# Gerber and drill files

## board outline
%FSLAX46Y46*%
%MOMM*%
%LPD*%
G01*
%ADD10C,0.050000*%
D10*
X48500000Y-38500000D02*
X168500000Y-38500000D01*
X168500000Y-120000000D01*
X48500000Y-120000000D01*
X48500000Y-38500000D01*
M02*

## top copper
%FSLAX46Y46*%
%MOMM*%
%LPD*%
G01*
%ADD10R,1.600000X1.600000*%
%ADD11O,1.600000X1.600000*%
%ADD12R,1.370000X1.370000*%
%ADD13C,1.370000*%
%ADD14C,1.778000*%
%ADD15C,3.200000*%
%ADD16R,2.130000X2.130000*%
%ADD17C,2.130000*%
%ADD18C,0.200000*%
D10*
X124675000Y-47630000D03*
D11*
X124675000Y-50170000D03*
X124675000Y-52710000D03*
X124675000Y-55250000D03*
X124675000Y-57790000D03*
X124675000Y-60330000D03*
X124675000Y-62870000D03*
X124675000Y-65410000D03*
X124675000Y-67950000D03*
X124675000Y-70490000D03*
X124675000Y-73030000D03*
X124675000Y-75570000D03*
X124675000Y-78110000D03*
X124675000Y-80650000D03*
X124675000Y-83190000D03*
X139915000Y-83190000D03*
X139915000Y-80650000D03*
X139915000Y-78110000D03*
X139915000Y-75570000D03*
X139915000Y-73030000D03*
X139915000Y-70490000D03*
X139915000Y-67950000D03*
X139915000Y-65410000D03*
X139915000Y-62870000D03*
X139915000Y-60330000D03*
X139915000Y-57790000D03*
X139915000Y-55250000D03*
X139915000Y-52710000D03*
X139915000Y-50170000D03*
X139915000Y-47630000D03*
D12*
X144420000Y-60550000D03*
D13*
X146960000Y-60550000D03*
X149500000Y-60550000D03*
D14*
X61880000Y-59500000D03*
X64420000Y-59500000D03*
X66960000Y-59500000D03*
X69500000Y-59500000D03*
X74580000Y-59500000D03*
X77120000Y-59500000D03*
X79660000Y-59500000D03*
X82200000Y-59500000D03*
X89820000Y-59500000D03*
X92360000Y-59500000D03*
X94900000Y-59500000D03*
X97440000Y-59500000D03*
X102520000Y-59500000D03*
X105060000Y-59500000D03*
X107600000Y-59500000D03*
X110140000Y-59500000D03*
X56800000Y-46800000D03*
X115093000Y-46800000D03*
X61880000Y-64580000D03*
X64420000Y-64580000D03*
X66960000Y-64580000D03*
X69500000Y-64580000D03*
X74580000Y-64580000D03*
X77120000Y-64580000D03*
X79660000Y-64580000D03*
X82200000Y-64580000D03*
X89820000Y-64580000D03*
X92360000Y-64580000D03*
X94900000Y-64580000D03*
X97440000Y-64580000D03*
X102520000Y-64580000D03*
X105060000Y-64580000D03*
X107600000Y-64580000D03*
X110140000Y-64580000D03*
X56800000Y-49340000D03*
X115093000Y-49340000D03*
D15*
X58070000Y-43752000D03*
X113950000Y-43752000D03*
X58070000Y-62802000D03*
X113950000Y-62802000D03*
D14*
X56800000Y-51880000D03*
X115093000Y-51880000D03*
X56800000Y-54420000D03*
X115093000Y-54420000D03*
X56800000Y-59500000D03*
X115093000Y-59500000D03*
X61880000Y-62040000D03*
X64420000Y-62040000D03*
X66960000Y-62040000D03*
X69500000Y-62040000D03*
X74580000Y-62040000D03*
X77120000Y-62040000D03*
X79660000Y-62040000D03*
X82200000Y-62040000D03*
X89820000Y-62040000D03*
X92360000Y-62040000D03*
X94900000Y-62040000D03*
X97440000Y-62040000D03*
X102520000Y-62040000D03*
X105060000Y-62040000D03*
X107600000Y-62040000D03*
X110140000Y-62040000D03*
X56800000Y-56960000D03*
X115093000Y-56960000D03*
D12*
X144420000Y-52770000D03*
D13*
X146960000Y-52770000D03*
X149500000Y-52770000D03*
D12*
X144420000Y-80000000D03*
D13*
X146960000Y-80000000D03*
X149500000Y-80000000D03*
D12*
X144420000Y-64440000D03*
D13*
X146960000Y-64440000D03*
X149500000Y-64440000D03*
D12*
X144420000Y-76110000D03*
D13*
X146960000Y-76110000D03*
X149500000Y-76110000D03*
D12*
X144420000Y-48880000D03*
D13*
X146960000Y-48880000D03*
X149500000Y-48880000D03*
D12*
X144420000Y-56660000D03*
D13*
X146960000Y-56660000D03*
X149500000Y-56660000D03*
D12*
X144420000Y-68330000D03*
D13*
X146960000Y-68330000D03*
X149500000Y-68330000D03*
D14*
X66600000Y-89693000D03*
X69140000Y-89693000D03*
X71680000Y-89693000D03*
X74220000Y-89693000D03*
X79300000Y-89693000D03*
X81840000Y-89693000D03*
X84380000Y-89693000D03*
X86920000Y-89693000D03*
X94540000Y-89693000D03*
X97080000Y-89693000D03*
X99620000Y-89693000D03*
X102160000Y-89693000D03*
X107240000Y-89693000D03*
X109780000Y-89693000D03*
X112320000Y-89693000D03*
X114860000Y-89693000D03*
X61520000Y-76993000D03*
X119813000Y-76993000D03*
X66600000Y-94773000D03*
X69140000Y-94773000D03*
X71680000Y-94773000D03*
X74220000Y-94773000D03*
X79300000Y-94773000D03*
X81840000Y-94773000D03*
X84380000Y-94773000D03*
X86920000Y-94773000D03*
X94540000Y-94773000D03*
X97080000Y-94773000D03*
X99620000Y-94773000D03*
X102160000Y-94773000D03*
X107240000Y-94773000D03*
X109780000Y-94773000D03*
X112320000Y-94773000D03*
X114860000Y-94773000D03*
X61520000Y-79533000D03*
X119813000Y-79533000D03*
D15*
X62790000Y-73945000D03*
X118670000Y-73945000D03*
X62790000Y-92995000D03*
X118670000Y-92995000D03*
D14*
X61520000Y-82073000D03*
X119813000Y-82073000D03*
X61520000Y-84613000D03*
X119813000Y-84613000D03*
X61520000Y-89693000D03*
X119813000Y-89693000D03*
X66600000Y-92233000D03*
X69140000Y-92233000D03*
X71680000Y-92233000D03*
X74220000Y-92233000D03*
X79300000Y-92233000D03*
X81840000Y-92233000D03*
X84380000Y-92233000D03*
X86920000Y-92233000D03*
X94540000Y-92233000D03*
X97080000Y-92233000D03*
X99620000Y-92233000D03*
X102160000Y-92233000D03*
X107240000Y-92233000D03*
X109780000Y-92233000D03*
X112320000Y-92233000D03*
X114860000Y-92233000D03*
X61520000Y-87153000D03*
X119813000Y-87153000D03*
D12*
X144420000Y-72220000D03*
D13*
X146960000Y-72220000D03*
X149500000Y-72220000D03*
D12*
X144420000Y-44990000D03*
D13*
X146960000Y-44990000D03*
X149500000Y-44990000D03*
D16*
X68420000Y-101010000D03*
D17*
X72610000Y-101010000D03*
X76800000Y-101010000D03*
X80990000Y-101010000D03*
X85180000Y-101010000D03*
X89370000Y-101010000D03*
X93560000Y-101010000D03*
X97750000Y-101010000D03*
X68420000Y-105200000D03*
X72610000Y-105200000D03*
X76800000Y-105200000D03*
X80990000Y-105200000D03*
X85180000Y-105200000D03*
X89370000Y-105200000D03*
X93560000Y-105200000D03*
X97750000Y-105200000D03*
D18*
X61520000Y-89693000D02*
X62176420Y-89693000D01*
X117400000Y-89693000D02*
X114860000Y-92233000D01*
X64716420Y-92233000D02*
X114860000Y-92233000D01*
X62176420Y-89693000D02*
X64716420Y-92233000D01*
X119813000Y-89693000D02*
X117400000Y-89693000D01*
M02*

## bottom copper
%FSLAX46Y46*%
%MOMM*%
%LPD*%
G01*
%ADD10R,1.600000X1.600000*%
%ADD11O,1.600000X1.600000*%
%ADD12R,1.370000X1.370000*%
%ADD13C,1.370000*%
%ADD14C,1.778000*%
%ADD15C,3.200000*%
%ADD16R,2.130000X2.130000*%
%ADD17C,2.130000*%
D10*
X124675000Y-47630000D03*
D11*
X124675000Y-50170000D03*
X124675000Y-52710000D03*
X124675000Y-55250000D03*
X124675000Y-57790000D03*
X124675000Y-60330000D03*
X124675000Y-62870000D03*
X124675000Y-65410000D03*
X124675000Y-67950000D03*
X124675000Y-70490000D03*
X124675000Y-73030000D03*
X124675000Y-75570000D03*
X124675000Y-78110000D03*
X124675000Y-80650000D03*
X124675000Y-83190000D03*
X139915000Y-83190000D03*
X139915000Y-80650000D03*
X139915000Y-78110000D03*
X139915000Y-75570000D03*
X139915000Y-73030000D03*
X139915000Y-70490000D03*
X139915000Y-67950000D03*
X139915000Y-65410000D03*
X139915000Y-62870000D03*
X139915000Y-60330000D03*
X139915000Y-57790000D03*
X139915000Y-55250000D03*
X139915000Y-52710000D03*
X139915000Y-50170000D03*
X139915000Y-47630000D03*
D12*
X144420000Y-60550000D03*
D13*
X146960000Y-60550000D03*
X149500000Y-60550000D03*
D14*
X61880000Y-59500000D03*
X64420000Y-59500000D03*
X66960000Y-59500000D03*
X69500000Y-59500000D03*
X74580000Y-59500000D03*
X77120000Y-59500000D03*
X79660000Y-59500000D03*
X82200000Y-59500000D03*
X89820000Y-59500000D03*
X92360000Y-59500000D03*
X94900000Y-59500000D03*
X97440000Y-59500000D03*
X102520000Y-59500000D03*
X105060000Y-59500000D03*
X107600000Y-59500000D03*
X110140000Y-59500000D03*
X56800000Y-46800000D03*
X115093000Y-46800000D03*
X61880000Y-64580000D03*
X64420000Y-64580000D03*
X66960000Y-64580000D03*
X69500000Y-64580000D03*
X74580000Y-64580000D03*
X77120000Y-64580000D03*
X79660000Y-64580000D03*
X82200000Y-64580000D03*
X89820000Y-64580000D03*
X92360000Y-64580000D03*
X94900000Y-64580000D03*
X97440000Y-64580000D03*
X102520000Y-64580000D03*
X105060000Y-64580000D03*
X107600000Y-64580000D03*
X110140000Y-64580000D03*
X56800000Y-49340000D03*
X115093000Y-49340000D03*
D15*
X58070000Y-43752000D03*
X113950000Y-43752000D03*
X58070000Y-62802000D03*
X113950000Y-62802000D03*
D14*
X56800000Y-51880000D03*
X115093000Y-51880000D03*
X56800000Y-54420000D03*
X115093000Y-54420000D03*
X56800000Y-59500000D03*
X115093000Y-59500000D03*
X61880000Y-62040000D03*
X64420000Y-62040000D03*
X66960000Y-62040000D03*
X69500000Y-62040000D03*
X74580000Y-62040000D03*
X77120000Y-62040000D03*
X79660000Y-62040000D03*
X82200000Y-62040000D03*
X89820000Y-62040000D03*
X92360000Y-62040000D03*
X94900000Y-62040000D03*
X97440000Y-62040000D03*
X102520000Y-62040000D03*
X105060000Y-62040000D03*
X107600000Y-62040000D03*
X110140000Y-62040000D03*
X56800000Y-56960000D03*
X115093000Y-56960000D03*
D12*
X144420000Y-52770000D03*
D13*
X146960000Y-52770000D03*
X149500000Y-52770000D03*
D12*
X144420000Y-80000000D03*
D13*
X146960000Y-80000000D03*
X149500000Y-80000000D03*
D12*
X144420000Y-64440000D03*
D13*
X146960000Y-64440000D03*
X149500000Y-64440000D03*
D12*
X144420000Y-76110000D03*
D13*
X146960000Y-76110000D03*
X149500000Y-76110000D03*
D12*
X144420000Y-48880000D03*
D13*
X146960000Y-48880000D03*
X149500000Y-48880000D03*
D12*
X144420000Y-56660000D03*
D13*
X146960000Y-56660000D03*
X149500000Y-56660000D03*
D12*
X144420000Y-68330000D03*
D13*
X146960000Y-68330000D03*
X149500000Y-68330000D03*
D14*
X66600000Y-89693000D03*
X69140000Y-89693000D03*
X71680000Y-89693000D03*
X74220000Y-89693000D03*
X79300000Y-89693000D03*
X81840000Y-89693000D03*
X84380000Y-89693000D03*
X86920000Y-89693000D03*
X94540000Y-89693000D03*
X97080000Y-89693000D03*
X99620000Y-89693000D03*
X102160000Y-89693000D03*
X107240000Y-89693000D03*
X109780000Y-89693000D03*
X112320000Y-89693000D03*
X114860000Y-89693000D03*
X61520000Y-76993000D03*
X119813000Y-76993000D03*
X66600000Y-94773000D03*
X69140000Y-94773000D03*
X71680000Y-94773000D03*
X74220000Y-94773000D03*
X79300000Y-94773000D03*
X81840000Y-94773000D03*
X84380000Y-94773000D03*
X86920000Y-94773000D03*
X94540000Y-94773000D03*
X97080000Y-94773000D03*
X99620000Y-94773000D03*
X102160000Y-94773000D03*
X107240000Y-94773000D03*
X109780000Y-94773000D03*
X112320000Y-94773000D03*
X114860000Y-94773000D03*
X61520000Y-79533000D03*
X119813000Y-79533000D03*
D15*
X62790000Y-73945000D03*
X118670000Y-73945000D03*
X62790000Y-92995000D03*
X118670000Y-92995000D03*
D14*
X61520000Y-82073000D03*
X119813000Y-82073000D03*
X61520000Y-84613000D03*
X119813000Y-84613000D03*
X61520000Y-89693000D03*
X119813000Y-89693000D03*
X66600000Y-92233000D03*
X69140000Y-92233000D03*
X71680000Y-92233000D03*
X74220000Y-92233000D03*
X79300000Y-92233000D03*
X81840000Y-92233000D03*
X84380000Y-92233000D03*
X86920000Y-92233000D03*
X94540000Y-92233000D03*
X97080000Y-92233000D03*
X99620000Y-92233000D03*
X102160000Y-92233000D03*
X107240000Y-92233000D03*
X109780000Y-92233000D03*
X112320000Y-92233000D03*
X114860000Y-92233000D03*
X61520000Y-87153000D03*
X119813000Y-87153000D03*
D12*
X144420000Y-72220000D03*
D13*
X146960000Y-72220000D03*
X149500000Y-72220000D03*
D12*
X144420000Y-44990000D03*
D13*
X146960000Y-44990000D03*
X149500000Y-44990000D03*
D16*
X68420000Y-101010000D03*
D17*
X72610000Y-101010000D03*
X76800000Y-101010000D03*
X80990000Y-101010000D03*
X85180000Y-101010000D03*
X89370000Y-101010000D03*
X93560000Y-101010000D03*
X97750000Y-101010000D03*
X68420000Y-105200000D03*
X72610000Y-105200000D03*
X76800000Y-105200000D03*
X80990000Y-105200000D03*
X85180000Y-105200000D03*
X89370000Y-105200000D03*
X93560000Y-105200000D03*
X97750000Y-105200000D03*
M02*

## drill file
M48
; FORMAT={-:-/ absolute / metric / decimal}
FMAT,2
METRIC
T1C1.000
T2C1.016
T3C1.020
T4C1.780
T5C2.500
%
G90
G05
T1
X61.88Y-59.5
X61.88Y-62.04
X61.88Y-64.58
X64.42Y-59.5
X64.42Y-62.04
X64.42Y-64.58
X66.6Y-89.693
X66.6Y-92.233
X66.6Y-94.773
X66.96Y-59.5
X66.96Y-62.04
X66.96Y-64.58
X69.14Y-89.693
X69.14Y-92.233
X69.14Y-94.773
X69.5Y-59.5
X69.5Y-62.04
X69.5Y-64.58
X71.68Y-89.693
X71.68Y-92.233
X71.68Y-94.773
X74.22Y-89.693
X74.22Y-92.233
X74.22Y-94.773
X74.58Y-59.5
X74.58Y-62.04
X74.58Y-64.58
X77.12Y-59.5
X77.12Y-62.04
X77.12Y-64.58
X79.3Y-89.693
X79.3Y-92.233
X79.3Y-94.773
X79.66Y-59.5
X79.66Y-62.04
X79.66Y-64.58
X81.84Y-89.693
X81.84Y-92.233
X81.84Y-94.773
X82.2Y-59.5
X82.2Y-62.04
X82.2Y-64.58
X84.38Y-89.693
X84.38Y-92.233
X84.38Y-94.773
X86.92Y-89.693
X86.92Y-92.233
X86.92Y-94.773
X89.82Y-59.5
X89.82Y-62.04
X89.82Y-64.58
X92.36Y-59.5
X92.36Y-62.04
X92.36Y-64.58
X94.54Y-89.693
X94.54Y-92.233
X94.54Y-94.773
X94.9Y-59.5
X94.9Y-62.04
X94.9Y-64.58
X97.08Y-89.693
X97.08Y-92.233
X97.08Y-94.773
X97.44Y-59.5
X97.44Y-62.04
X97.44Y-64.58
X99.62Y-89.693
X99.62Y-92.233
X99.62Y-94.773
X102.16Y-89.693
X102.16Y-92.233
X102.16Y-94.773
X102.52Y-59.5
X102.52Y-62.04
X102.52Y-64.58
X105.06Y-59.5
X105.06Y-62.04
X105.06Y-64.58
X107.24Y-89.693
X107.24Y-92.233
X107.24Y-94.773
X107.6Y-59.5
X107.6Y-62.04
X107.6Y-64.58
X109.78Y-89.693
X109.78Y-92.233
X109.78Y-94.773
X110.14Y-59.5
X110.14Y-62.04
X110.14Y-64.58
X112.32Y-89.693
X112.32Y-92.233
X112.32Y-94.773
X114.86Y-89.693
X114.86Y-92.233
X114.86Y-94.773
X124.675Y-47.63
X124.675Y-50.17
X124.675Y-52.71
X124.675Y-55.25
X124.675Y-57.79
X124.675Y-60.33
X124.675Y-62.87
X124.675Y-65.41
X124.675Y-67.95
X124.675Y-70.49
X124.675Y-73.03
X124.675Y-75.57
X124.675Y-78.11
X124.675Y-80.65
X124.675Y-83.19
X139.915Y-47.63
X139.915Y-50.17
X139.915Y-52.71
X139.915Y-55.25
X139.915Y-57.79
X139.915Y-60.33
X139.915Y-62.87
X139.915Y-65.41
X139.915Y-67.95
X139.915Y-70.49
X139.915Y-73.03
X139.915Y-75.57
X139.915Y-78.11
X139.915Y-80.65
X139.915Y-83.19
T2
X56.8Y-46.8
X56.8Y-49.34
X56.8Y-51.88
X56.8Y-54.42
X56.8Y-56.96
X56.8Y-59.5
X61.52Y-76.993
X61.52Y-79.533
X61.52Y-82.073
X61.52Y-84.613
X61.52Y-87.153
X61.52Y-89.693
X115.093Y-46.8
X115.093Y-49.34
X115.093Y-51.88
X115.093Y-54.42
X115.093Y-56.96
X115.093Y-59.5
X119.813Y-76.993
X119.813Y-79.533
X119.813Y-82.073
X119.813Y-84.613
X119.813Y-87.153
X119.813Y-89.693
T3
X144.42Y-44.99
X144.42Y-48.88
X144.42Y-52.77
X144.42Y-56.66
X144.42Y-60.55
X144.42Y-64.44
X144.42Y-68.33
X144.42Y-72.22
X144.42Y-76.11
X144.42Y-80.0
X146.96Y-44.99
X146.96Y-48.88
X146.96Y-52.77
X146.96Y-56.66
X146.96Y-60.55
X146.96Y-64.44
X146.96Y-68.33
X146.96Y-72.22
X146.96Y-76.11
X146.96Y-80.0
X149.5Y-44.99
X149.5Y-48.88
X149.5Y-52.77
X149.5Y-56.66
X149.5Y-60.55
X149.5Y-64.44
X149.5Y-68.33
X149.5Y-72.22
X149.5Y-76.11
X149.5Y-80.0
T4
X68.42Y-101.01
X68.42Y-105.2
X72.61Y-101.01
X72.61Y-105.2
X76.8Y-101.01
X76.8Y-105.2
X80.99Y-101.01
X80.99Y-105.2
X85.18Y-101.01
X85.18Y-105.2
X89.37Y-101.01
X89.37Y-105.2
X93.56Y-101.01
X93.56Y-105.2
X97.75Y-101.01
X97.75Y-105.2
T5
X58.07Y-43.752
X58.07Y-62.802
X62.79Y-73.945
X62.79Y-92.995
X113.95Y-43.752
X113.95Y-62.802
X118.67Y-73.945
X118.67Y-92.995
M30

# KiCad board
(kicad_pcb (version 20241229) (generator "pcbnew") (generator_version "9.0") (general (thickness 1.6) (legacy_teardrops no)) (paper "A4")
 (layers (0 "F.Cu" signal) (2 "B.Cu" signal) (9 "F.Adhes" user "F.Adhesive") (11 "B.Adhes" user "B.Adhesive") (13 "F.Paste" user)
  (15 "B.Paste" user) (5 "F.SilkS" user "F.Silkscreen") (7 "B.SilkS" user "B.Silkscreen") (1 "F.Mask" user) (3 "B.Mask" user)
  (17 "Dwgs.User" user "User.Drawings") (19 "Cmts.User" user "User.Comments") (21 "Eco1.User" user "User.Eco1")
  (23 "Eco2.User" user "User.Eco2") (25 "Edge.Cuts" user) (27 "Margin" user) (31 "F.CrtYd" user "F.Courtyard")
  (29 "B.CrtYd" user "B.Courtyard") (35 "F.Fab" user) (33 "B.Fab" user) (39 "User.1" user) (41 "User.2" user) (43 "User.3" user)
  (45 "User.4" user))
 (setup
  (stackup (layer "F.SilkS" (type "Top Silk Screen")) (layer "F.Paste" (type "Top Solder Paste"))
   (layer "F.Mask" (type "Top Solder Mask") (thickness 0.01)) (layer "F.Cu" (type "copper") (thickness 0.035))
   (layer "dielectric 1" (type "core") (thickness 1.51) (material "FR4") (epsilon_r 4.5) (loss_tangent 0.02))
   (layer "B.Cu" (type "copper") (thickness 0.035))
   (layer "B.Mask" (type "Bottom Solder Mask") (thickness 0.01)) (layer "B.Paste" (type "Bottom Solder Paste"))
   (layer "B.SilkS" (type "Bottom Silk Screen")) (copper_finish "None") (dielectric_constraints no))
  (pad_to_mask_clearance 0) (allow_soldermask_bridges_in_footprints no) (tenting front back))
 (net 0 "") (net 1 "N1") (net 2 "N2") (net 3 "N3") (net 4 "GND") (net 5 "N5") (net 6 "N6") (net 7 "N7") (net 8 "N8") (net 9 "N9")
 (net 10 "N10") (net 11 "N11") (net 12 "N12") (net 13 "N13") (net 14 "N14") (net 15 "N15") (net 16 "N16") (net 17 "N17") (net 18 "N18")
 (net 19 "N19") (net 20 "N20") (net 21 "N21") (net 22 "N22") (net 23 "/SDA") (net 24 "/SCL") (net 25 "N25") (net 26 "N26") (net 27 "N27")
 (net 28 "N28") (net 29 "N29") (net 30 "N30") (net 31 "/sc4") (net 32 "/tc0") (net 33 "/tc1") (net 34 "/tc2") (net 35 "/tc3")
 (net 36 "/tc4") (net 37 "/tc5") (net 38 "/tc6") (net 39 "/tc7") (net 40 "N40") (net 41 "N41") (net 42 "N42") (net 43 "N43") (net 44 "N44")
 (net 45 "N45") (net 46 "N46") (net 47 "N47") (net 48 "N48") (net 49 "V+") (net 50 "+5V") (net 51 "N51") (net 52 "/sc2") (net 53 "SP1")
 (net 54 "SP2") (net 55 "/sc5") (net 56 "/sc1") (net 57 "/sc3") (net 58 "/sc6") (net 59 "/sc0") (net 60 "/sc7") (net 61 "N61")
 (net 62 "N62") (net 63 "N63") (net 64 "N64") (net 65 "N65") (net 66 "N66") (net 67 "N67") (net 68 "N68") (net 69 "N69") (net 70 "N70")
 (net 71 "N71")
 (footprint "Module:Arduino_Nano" (layer "F.Cu") (at 124.675 47.63)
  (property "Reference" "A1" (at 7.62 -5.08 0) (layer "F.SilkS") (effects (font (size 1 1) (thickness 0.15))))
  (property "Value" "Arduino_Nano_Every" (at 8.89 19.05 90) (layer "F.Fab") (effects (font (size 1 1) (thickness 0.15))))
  (pad "1" thru_hole rect (at 0 0) (size 1.6 1.6) (drill 1) (layers "*.Cu" "*.Mask") (remove_unused_layers no) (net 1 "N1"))
  (pad "2" thru_hole oval (at 0 2.54) (size 1.6 1.6) (drill 1) (layers "*.Cu" "*.Mask") (remove_unused_layers no) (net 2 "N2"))
  (pad "3" thru_hole oval (at 0 5.08) (size 1.6 1.6) (drill 1) (layers "*.Cu" "*.Mask") (remove_unused_layers no) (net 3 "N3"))
  (pad "4" thru_hole oval (at 0 7.62) (size 1.6 1.6) (drill 1) (layers "*.Cu" "*.Mask") (remove_unused_layers no) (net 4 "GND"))
  (pad "5" thru_hole oval (at 0 10.16) (size 1.6 1.6) (drill 1) (layers "*.Cu" "*.Mask") (remove_unused_layers no) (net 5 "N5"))
  (pad "6" thru_hole oval (at 0 12.7) (size 1.6 1.6) (drill 1) (layers "*.Cu" "*.Mask") (remove_unused_layers no) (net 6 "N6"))
  (pad "7" thru_hole oval (at 0 15.24) (size 1.6 1.6) (drill 1) (layers "*.Cu" "*.Mask") (remove_unused_layers no) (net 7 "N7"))
  (pad "8" thru_hole oval (at 0 17.78) (size 1.6 1.6) (drill 1) (layers "*.Cu" "*.Mask") (remove_unused_layers no) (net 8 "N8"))
  (pad "9" thru_hole oval (at 0 20.32) (size 1.6 1.6) (drill 1) (layers "*.Cu" "*.Mask") (remove_unused_layers no) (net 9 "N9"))
  (pad "10" thru_hole oval (at 0 22.86) (size 1.6 1.6) (drill 1) (layers "*.Cu" "*.Mask") (remove_unused_layers no) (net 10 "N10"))
  (pad "11" thru_hole oval (at 0 25.4) (size 1.6 1.6) (drill 1) (layers "*.Cu" "*.Mask") (remove_unused_layers no) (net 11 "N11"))
  (pad "12" thru_hole oval (at 0 27.94) (size 1.6 1.6) (drill 1) (layers "*.Cu" "*.Mask") (remove_unused_layers no) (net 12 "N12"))
  (pad "13" thru_hole oval (at 0 30.48) (size 1.6 1.6) (drill 1) (layers "*.Cu" "*.Mask") (remove_unused_layers no) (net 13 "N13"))
  (pad "14" thru_hole oval (at 0 33.02) (size 1.6 1.6) (drill 1) (layers "*.Cu" "*.Mask") (remove_unused_layers no) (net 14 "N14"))
  (pad "15" thru_hole oval (at 0 35.56) (size 1.6 1.6) (drill 1) (layers "*.Cu" "*.Mask") (remove_unused_layers no) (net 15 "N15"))
  (pad "16" thru_hole oval (at 15.24 35.56) (size 1.6 1.6) (drill 1) (layers "*.Cu" "*.Mask") (remove_unused_layers no) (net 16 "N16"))
  (pad "17" thru_hole oval (at 15.24 33.02) (size 1.6 1.6) (drill 1) (layers "*.Cu" "*.Mask") (remove_unused_layers no) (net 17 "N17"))
  (pad "18" thru_hole oval (at 15.24 30.48) (size 1.6 1.6) (drill 1) (layers "*.Cu" "*.Mask") (remove_unused_layers no) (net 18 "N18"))
  (pad "19" thru_hole oval (at 15.24 27.94) (size 1.6 1.6) (drill 1) (layers "*.Cu" "*.Mask") (remove_unused_layers no) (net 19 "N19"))
  (pad "20" thru_hole oval (at 15.24 25.4) (size 1.6 1.6) (drill 1) (layers "*.Cu" "*.Mask") (remove_unused_layers no) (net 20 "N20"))
  (pad "21" thru_hole oval (at 15.24 22.86) (size 1.6 1.6) (drill 1) (layers "*.Cu" "*.Mask") (remove_unused_layers no) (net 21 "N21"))
  (pad "22" thru_hole oval (at 15.24 20.32) (size 1.6 1.6) (drill 1) (layers "*.Cu" "*.Mask") (remove_unused_layers no) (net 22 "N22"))
  (pad "23" thru_hole oval (at 15.24 17.78) (size 1.6 1.6) (drill 1) (layers "*.Cu" "*.Mask") (remove_unused_layers no) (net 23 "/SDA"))
  (pad "24" thru_hole oval (at 15.24 15.24) (size 1.6 1.6) (drill 1) (layers "*.Cu" "*.Mask") (remove_unused_layers no) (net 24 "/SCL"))
  (pad "25" thru_hole oval (at 15.24 12.7) (size 1.6 1.6) (drill 1) (layers "*.Cu" "*.Mask") (remove_unused_layers no) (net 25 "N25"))
  (pad "26" thru_hole oval (at 15.24 10.16) (size 1.6 1.6) (drill 1) (layers "*.Cu" "*.Mask") (remove_unused_layers no) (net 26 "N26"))
  (pad "27" thru_hole oval (at 15.24 7.62) (size 1.6 1.6) (drill 1) (layers "*.Cu" "*.Mask") (remove_unused_layers no) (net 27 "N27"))
  (pad "28" thru_hole oval (at 15.24 5.08) (size 1.6 1.6) (drill 1) (layers "*.Cu" "*.Mask") (remove_unused_layers no) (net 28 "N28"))
  (pad "29" thru_hole oval (at 15.24 2.54) (size 1.6 1.6) (drill 1) (layers "*.Cu" "*.Mask") (remove_unused_layers no) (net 4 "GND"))
  (pad "30" thru_hole oval (at 15.24 0) (size 1.6 1.6) (drill 1) (layers "*.Cu" "*.Mask") (remove_unused_layers no) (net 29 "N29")))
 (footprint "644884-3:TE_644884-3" (layer "F.Cu") (at 144.42 60.55)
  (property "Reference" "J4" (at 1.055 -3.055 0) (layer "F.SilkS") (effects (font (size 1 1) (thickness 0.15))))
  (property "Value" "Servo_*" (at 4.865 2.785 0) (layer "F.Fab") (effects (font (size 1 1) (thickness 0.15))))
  (pad "1" thru_hole rect (at 0 0) (size 1.37 1.37) (drill 1.02) (layers "*.Cu" "*.Mask") (remove_unused_layers no) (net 4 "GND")
   (solder_mask_margin 0.102))
  (pad "2" thru_hole circle (at 2.54 0) (size 1.37 1.37) (drill 1.02) (layers "*.Cu" "*.Mask") (remove_unused_layers no) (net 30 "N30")
   (solder_mask_margin 0.102))
  (pad "3" thru_hole circle (at 5.08 0) (size 1.37 1.37) (drill 1.02) (layers "*.Cu" "*.Mask") (remove_unused_layers no) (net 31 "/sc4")
   (solder_mask_margin 0.102)))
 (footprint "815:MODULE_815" (layer "F.Cu") (at 86.01 53.277)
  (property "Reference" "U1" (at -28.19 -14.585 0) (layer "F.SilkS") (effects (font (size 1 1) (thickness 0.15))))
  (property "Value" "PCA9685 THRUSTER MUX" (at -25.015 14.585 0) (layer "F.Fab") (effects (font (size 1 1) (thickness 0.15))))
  (pad "0" thru_hole circle (at -24.13 6.223) (size 1.778 1.778) (drill 1) (layers "*.Cu" "*.Mask") (remove_unused_layers no)
   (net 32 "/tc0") (solder_mask_margin 0.102))
  (pad "1" thru_hole circle (at -21.59 6.223) (size 1.778 1.778) (drill 1) (layers "*.Cu" "*.Mask") (remove_unused_layers no)
   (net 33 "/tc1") (solder_mask_margin 0.102))
  (pad "2" thru_hole circle (at -19.05 6.223) (size 1.778 1.778) (drill 1) (layers "*.Cu" "*.Mask") (remove_unused_layers no)
   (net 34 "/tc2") (solder_mask_margin 0.102))
  (pad "3" thru_hole circle (at -16.51 6.223) (size 1.778 1.778) (drill 1) (layers "*.Cu" "*.Mask") (remove_unused_layers no)
   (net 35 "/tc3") (solder_mask_margin 0.102))
  (pad "4" thru_hole circle (at -11.43 6.223) (size 1.778 1.778) (drill 1) (layers "*.Cu" "*.Mask") (remove_unused_layers no)
   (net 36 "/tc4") (solder_mask_margin 0.102))
  (pad "5" thru_hole circle (at -8.89 6.223) (size 1.778 1.778) (drill 1) (layers "*.Cu" "*.Mask") (remove_unused_layers no) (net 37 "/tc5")
   (solder_mask_margin 0.102))
  (pad "6" thru_hole circle (at -6.35 6.223) (size 1.778 1.778) (drill 1) (layers "*.Cu" "*.Mask") (remove_unused_layers no) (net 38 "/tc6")
   (solder_mask_margin 0.102))
  (pad "7" thru_hole circle (at -3.81 6.223) (size 1.778 1.778) (drill 1) (layers "*.Cu" "*.Mask") (remove_unused_layers no) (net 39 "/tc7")
   (solder_mask_margin 0.102))
  (pad "8" thru_hole circle (at 3.81 6.223) (size 1.778 1.778) (drill 1) (layers "*.Cu" "*.Mask") (remove_unused_layers no) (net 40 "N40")
   (solder_mask_margin 0.102))
  (pad "9" thru_hole circle (at 6.35 6.223) (size 1.778 1.778) (drill 1) (layers "*.Cu" "*.Mask") (remove_unused_layers no) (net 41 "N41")
   (solder_mask_margin 0.102))
  (pad "10" thru_hole circle (at 8.89 6.223) (size 1.778 1.778) (drill 1) (layers "*.Cu" "*.Mask") (remove_unused_layers no) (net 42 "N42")
   (solder_mask_margin 0.102))
  (pad "11" thru_hole circle (at 11.43 6.223) (size 1.778 1.778) (drill 1) (layers "*.Cu" "*.Mask") (remove_unused_layers no) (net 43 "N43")
   (solder_mask_margin 0.102))
  (pad "12" thru_hole circle (at 16.51 6.223) (size 1.778 1.778) (drill 1) (layers "*.Cu" "*.Mask") (remove_unused_layers no) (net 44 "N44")
   (solder_mask_margin 0.102))
  (pad "13" thru_hole circle (at 19.05 6.223) (size 1.778 1.778) (drill 1) (layers "*.Cu" "*.Mask") (remove_unused_layers no) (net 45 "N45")
   (solder_mask_margin 0.102))
  (pad "14" thru_hole circle (at 21.59 6.223) (size 1.778 1.778) (drill 1) (layers "*.Cu" "*.Mask") (remove_unused_layers no) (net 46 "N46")
   (solder_mask_margin 0.102))
  (pad "15" thru_hole circle (at 24.13 6.223) (size 1.778 1.778) (drill 1) (layers "*.Cu" "*.Mask") (remove_unused_layers no) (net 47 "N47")
   (solder_mask_margin 0.102))
  (pad "GND_1" thru_hole circle (at -29.21 -6.477) (size 1.778 1.778) (drill 1.016) (layers "*.Cu" "*.Mask") (remove_unused_layers no)
   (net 4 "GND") (solder_mask_margin 0.102))
  (pad "GND_2" thru_hole circle (at 29.083 -6.477) (size 1.778 1.778) (drill 1.016) (layers "*.Cu" "*.Mask") (remove_unused_layers no)
   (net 4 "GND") (solder_mask_margin 0.102))
  (pad "GND_3" thru_hole circle (at -24.13 11.303) (size 1.778 1.778) (drill 1) (layers "*.Cu" "*.Mask") (remove_unused_layers no)
   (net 4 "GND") (solder_mask_margin 0.102))
  (pad "GND_4" thru_hole circle (at -21.59 11.303) (size 1.778 1.778) (drill 1) (layers "*.Cu" "*.Mask") (remove_unused_layers no)
   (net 4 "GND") (solder_mask_margin 0.102))
  (pad "GND_5" thru_hole circle (at -19.05 11.303) (size 1.778 1.778) (drill 1) (layers "*.Cu" "*.Mask") (remove_unused_layers no)
   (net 4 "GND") (solder_mask_margin 0.102))
  (pad "GND_6" thru_hole circle (at -16.51 11.303) (size 1.778 1.778) (drill 1) (layers "*.Cu" "*.Mask") (remove_unused_layers no)
   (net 4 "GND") (solder_mask_margin 0.102))
  (pad "GND_7" thru_hole circle (at -11.43 11.303) (size 1.778 1.778) (drill 1) (layers "*.Cu" "*.Mask") (remove_unused_layers no)
   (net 4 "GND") (solder_mask_margin 0.102))
  (pad "GND_8" thru_hole circle (at -8.89 11.303) (size 1.778 1.778) (drill 1) (layers "*.Cu" "*.Mask") (remove_unused_layers no)
   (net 4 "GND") (solder_mask_margin 0.102))
  (pad "GND_9" thru_hole circle (at -6.35 11.303) (size 1.778 1.778) (drill 1) (layers "*.Cu" "*.Mask") (remove_unused_layers no)
   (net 4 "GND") (solder_mask_margin 0.102))
  (pad "GND_10" thru_hole circle (at -3.81 11.303) (size 1.778 1.778) (drill 1) (layers "*.Cu" "*.Mask") (remove_unused_layers no)
   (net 4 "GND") (solder_mask_margin 0.102))
  (pad "GND_11" thru_hole circle (at 3.81 11.303) (size 1.778 1.778) (drill 1) (layers "*.Cu" "*.Mask") (remove_unused_layers no)
   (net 4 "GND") (solder_mask_margin 0.102))
  (pad "GND_12" thru_hole circle (at 6.35 11.303) (size 1.778 1.778) (drill 1) (layers "*.Cu" "*.Mask") (remove_unused_layers no)
   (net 4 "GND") (solder_mask_margin 0.102))
  (pad "GND_13" thru_hole circle (at 8.89 11.303) (size 1.778 1.778) (drill 1) (layers "*.Cu" "*.Mask") (remove_unused_layers no)
   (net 4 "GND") (solder_mask_margin 0.102))
  (pad "GND_14" thru_hole circle (at 11.43 11.303) (size 1.778 1.778) (drill 1) (layers "*.Cu" "*.Mask") (remove_unused_layers no)
   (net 4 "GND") (solder_mask_margin 0.102))
  (pad "GND_15" thru_hole circle (at 16.51 11.303) (size 1.778 1.778) (drill 1) (layers "*.Cu" "*.Mask") (remove_unused_layers no)
   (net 4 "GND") (solder_mask_margin 0.102))
  (pad "GND_16" thru_hole circle (at 19.05 11.303) (size 1.778 1.778) (drill 1) (layers "*.Cu" "*.Mask") (remove_unused_layers no)
   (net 4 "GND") (solder_mask_margin 0.102))
  (pad "GND_17" thru_hole circle (at 21.59 11.303) (size 1.778 1.778) (drill 1) (layers "*.Cu" "*.Mask") (remove_unused_layers no)
   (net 4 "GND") (solder_mask_margin 0.102))
  (pad "GND_18" thru_hole circle (at 24.13 11.303) (size 1.778 1.778) (drill 1) (layers "*.Cu" "*.Mask") (remove_unused_layers no)
   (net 4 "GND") (solder_mask_margin 0.102))
  (pad "OE_1" thru_hole circle (at -29.21 -3.937) (size 1.778 1.778) (drill 1.016) (layers "*.Cu" "*.Mask") (remove_unused_layers no)
   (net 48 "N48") (solder_mask_margin 0.102))
  (pad "OE_2" thru_hole circle (at 29.083 -3.937) (size 1.778 1.778) (drill 1.016) (layers "*.Cu" "*.Mask") (remove_unused_layers no)
   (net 48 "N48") (solder_mask_margin 0.102))
  (pad "S1" thru_hole circle (at -27.94 -9.525) (size 3.2 3.2) (drill 2.5) (layers "*.Cu" "*.Mask") (remove_unused_layers no)
   (solder_mask_margin 0.102))
  (pad "S2" thru_hole circle (at 27.94 -9.525) (size 3.2 3.2) (drill 2.5) (layers "*.Cu" "*.Mask") (remove_unused_layers no)
   (solder_mask_margin 0.102))
  (pad "S3" thru_hole circle (at -27.94 9.525) (size 3.2 3.2) (drill 2.5) (layers "*.Cu" "*.Mask") (remove_unused_layers no)
   (solder_mask_margin 0.102))
  (pad "S4" thru_hole circle (at 27.94 9.525) (size 3.2 3.2) (drill 2.5) (layers "*.Cu" "*.Mask") (remove_unused_layers no)
   (solder_mask_margin 0.102))
  (pad "SCL_1" thru_hole circle (at -29.21 -1.397) (size 1.778 1.778) (drill 1.016) (layers "*.Cu" "*.Mask") (remove_unused_layers no)
   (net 24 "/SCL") (solder_mask_margin 0.102))
  (pad "SCL_2" thru_hole circle (at 29.083 -1.397) (size 1.778 1.778) (drill 1.016) (layers "*.Cu" "*.Mask") (remove_unused_layers no)
   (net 24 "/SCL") (solder_mask_margin 0.102))
  (pad "SDA_1" thru_hole circle (at -29.21 1.143) (size 1.778 1.778) (drill 1.016) (layers "*.Cu" "*.Mask") (remove_unused_layers no)
   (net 23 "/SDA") (solder_mask_margin 0.102))
  (pad "SDA_2" thru_hole circle (at 29.083 1.143) (size 1.778 1.778) (drill 1.016) (layers "*.Cu" "*.Mask") (remove_unused_layers no)
   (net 23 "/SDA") (solder_mask_margin 0.102))
  (pad "V+_1" thru_hole circle (at -29.21 6.223) (size 1.778 1.778) (drill 1.016) (layers "*.Cu" "*.Mask") (remove_unused_layers no)
   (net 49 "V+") (solder_mask_margin 0.102))
  (pad "V+_2" thru_hole circle (at 29.083 6.223) (size 1.778 1.778) (drill 1.016) (layers "*.Cu" "*.Mask") (remove_unused_layers no)
   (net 49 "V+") (solder_mask_margin 0.102))
  (pad "V+_3" thru_hole circle (at -24.13 8.763) (size 1.778 1.778) (drill 1) (layers "*.Cu" "*.Mask") (remove_unused_layers no)
   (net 49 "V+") (solder_mask_margin 0.102))
  (pad "V+_4" thru_hole circle (at -21.59 8.763) (size 1.778 1.778) (drill 1) (layers "*.Cu" "*.Mask") (remove_unused_layers no)
   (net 49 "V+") (solder_mask_margin 0.102))
  (pad "V+_5" thru_hole circle (at -19.05 8.763) (size 1.778 1.778) (drill 1) (layers "*.Cu" "*.Mask") (remove_unused_layers no)
   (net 49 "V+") (solder_mask_margin 0.102))
  (pad "V+_6" thru_hole circle (at -16.51 8.763) (size 1.778 1.778) (drill 1) (layers "*.Cu" "*.Mask") (remove_unused_layers no)
   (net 49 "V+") (solder_mask_margin 0.102))
  (pad "V+_7" thru_hole circle (at -11.43 8.763) (size 1.778 1.778) (drill 1) (layers "*.Cu" "*.Mask") (remove_unused_layers no)
   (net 49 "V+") (solder_mask_margin 0.102))
  (pad "V+_8" thru_hole circle (at -8.89 8.763) (size 1.778 1.778) (drill 1) (layers "*.Cu" "*.Mask") (remove_unused_layers no)
   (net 49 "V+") (solder_mask_margin 0.102))
  (pad "V+_9" thru_hole circle (at -6.35 8.763) (size 1.778 1.778) (drill 1) (layers "*.Cu" "*.Mask") (remove_unused_layers no)
   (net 49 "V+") (solder_mask_margin 0.102))
  (pad "V+_10" thru_hole circle (at -3.81 8.763) (size 1.778 1.778) (drill 1) (layers "*.Cu" "*.Mask") (remove_unused_layers no)
   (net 49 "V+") (solder_mask_margin 0.102))
  (pad "V+_11" thru_hole circle (at 3.81 8.763) (size 1.778 1.778) (drill 1) (layers "*.Cu" "*.Mask") (remove_unused_layers no)
   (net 49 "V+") (solder_mask_margin 0.102))
  (pad "V+_12" thru_hole circle (at 6.35 8.763) (size 1.778 1.778) (drill 1) (layers "*.Cu" "*.Mask") (remove_unused_layers no)
   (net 49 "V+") (solder_mask_margin 0.102))
  (pad "V+_13" thru_hole circle (at 8.89 8.763) (size 1.778 1.778) (drill 1) (layers "*.Cu" "*.Mask") (remove_unused_layers no)
   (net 49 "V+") (solder_mask_margin 0.102))
  (pad "V+_14" thru_hole circle (at 11.43 8.763) (size 1.778 1.778) (drill 1) (layers "*.Cu" "*.Mask") (remove_unused_layers no)
   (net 49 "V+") (solder_mask_margin 0.102))
  (pad "V+_15" thru_hole circle (at 16.51 8.763) (size 1.778 1.778) (drill 1) (layers "*.Cu" "*.Mask") (remove_unused_layers no)
   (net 49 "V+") (solder_mask_margin 0.102))
  (pad "V+_16" thru_hole circle (at 19.05 8.763) (size 1.778 1.778) (drill 1) (layers "*.Cu" "*.Mask") (remove_unused_layers no)
   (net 49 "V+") (solder_mask_margin 0.102))
  (pad "V+_17" thru_hole circle (at 21.59 8.763) (size 1.778 1.778) (drill 1) (layers "*.Cu" "*.Mask") (remove_unused_layers no)
   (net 49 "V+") (solder_mask_margin 0.102))
  (pad "V+_18" thru_hole circle (at 24.13 8.763) (size 1.778 1.778) (drill 1) (layers "*.Cu" "*.Mask") (remove_unused_layers no)
   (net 49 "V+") (solder_mask_margin 0.102))
  (pad "VCC_1" thru_hole circle (at -29.21 3.683) (size 1.778 1.778) (drill 1.016) (layers "*.Cu" "*.Mask") (remove_unused_layers no)
   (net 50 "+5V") (solder_mask_margin 0.102))
  (pad "VCC_2" thru_hole circle (at 29.083 3.683) (size 1.778 1.778) (drill 1.016) (layers "*.Cu" "*.Mask") (remove_unused_layers no)
   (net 50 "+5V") (solder_mask_margin 0.102)))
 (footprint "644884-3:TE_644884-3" (layer "F.Cu") (at 144.42 52.77)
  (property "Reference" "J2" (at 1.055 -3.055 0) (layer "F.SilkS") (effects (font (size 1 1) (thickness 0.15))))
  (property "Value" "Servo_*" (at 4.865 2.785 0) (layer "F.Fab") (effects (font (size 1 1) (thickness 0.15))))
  (pad "1" thru_hole rect (at 0 0) (size 1.37 1.37) (drill 1.02) (layers "*.Cu" "*.Mask") (remove_unused_layers no) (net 4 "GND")
   (solder_mask_margin 0.102))
  (pad "2" thru_hole circle (at 2.54 0) (size 1.37 1.37) (drill 1.02) (layers "*.Cu" "*.Mask") (remove_unused_layers no) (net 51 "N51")
   (solder_mask_margin 0.102))
  (pad "3" thru_hole circle (at 5.08 0) (size 1.37 1.37) (drill 1.02) (layers "*.Cu" "*.Mask") (remove_unused_layers no) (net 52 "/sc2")
   (solder_mask_margin 0.102)))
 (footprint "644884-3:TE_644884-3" (layer "F.Cu") (at 144.42 80)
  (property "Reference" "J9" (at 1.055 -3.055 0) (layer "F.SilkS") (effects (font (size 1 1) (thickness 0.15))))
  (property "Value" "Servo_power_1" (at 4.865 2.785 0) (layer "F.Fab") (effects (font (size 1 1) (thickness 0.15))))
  (pad "1" thru_hole rect (at 0 0) (size 1.37 1.37) (drill 1.02) (layers "*.Cu" "*.Mask") (remove_unused_layers no) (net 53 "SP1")
   (solder_mask_margin 0.102))
  (pad "2" thru_hole circle (at 2.54 0) (size 1.37 1.37) (drill 1.02) (layers "*.Cu" "*.Mask") (remove_unused_layers no) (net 30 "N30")
   (solder_mask_margin 0.102))
  (pad "3" thru_hole circle (at 5.08 0) (size 1.37 1.37) (drill 1.02) (layers "*.Cu" "*.Mask") (remove_unused_layers no) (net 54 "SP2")
   (solder_mask_margin 0.102)))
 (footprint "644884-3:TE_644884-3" (layer "F.Cu") (at 144.42 64.44)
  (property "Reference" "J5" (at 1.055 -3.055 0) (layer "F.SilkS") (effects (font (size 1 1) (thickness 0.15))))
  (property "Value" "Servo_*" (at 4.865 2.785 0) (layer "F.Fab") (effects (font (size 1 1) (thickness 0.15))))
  (pad "1" thru_hole rect (at 0 0) (size 1.37 1.37) (drill 1.02) (layers "*.Cu" "*.Mask") (remove_unused_layers no) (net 4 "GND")
   (solder_mask_margin 0.102))
  (pad "2" thru_hole circle (at 2.54 0) (size 1.37 1.37) (drill 1.02) (layers "*.Cu" "*.Mask") (remove_unused_layers no) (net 30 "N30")
   (solder_mask_margin 0.102))
  (pad "3" thru_hole circle (at 5.08 0) (size 1.37 1.37) (drill 1.02) (layers "*.Cu" "*.Mask") (remove_unused_layers no) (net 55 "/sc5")
   (solder_mask_margin 0.102)))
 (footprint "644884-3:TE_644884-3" (layer "F.Cu") (at 144.42 76.11)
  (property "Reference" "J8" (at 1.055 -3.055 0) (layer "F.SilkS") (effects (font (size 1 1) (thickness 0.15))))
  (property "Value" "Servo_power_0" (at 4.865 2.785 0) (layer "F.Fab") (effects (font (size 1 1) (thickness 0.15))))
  (pad "1" thru_hole rect (at 0 0) (size 1.37 1.37) (drill 1.02) (layers "*.Cu" "*.Mask") (remove_unused_layers no) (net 53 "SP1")
   (solder_mask_margin 0.102))
  (pad "2" thru_hole circle (at 2.54 0) (size 1.37 1.37) (drill 1.02) (layers "*.Cu" "*.Mask") (remove_unused_layers no) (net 51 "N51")
   (solder_mask_margin 0.102))
  (pad "3" thru_hole circle (at 5.08 0) (size 1.37 1.37) (drill 1.02) (layers "*.Cu" "*.Mask") (remove_unused_layers no) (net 54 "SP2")
   (solder_mask_margin 0.102)))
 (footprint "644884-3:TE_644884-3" (layer "F.Cu") (at 144.42 48.88)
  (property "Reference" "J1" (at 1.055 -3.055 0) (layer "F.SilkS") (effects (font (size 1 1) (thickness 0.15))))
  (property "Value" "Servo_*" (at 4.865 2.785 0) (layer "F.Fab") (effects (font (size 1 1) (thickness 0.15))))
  (pad "1" thru_hole rect (at 0 0) (size 1.37 1.37) (drill 1.02) (layers "*.Cu" "*.Mask") (remove_unused_layers no) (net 4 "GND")
   (solder_mask_margin 0.102))
  (pad "2" thru_hole circle (at 2.54 0) (size 1.37 1.37) (drill 1.02) (layers "*.Cu" "*.Mask") (remove_unused_layers no) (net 51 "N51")
   (solder_mask_margin 0.102))
  (pad "3" thru_hole circle (at 5.08 0) (size 1.37 1.37) (drill 1.02) (layers "*.Cu" "*.Mask") (remove_unused_layers no) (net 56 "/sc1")
   (solder_mask_margin 0.102)))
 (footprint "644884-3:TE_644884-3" (layer "F.Cu") (at 144.42 56.66)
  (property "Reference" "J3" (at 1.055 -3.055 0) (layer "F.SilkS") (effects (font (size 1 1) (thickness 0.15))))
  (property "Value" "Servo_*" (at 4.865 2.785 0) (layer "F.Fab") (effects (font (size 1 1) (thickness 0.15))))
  (pad "1" thru_hole rect (at 0 0) (size 1.37 1.37) (drill 1.02) (layers "*.Cu" "*.Mask") (remove_unused_layers no) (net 4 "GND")
   (solder_mask_margin 0.102))
  (pad "2" thru_hole circle (at 2.54 0) (size 1.37 1.37) (drill 1.02) (layers "*.Cu" "*.Mask") (remove_unused_layers no) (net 51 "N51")
   (solder_mask_margin 0.102))
  (pad "3" thru_hole circle (at 5.08 0) (size 1.37 1.37) (drill 1.02) (layers "*.Cu" "*.Mask") (remove_unused_layers no) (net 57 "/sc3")
   (solder_mask_margin 0.102)))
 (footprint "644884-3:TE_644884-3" (layer "F.Cu") (at 144.42 68.33)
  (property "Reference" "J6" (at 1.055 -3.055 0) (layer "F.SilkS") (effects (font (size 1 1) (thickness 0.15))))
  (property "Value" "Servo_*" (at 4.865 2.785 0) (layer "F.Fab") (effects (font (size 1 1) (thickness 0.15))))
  (pad "1" thru_hole rect (at 0 0) (size 1.37 1.37) (drill 1.02) (layers "*.Cu" "*.Mask") (remove_unused_layers no) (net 4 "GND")
   (solder_mask_margin 0.102))
  (pad "2" thru_hole circle (at 2.54 0) (size 1.37 1.37) (drill 1.02) (layers "*.Cu" "*.Mask") (remove_unused_layers no) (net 30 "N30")
   (solder_mask_margin 0.102))
  (pad "3" thru_hole circle (at 5.08 0) (size 1.37 1.37) (drill 1.02) (layers "*.Cu" "*.Mask") (remove_unused_layers no) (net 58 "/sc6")
   (solder_mask_margin 0.102)))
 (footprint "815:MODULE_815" (layer "F.Cu") (at 90.73 83.47)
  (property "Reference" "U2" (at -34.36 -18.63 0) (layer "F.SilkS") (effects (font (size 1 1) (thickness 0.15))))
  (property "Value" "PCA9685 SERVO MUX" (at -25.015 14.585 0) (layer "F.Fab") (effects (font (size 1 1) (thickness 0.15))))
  (pad "0" thru_hole circle (at -24.13 6.223) (size 1.778 1.778) (drill 1) (layers "*.Cu" "*.Mask") (remove_unused_layers no)
   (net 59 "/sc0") (solder_mask_margin 0.102))
  (pad "1" thru_hole circle (at -21.59 6.223) (size 1.778 1.778) (drill 1) (layers "*.Cu" "*.Mask") (remove_unused_layers no)
   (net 56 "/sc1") (solder_mask_margin 0.102))
  (pad "2" thru_hole circle (at -19.05 6.223) (size 1.778 1.778) (drill 1) (layers "*.Cu" "*.Mask") (remove_unused_layers no)
   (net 52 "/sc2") (solder_mask_margin 0.102))
  (pad "3" thru_hole circle (at -16.51 6.223) (size 1.778 1.778) (drill 1) (layers "*.Cu" "*.Mask") (remove_unused_layers no)
   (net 57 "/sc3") (solder_mask_margin 0.102))
  (pad "4" thru_hole circle (at -11.43 6.223) (size 1.778 1.778) (drill 1) (layers "*.Cu" "*.Mask") (remove_unused_layers no)
   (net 31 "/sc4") (solder_mask_margin 0.102))
  (pad "5" thru_hole circle (at -8.89 6.223) (size 1.778 1.778) (drill 1) (layers "*.Cu" "*.Mask") (remove_unused_layers no) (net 55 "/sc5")
   (solder_mask_margin 0.102))
  (pad "6" thru_hole circle (at -6.35 6.223) (size 1.778 1.778) (drill 1) (layers "*.Cu" "*.Mask") (remove_unused_layers no) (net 58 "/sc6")
   (solder_mask_margin 0.102))
  (pad "7" thru_hole circle (at -3.81 6.223) (size 1.778 1.778) (drill 1) (layers "*.Cu" "*.Mask") (remove_unused_layers no) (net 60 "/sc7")
   (solder_mask_margin 0.102))
  (pad "8" thru_hole circle (at 3.81 6.223) (size 1.778 1.778) (drill 1) (layers "*.Cu" "*.Mask") (remove_unused_layers no) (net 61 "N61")
   (solder_mask_margin 0.102))
  (pad "9" thru_hole circle (at 6.35 6.223) (size 1.778 1.778) (drill 1) (layers "*.Cu" "*.Mask") (remove_unused_layers no) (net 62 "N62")
   (solder_mask_margin 0.102))
  (pad "10" thru_hole circle (at 8.89 6.223) (size 1.778 1.778) (drill 1) (layers "*.Cu" "*.Mask") (remove_unused_layers no) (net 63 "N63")
   (solder_mask_margin 0.102))
  (pad "11" thru_hole circle (at 11.43 6.223) (size 1.778 1.778) (drill 1) (layers "*.Cu" "*.Mask") (remove_unused_layers no) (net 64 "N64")
   (solder_mask_margin 0.102))
  (pad "12" thru_hole circle (at 16.51 6.223) (size 1.778 1.778) (drill 1) (layers "*.Cu" "*.Mask") (remove_unused_layers no) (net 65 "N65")
   (solder_mask_margin 0.102))
  (pad "13" thru_hole circle (at 19.05 6.223) (size 1.778 1.778) (drill 1) (layers "*.Cu" "*.Mask") (remove_unused_layers no) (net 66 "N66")
   (solder_mask_margin 0.102))
  (pad "14" thru_hole circle (at 21.59 6.223) (size 1.778 1.778) (drill 1) (layers "*.Cu" "*.Mask") (remove_unused_layers no) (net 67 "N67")
   (solder_mask_margin 0.102))
  (pad "15" thru_hole circle (at 24.13 6.223) (size 1.778 1.778) (drill 1) (layers "*.Cu" "*.Mask") (remove_unused_layers no) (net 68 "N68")
   (solder_mask_margin 0.102))
  (pad "GND_1" thru_hole circle (at -29.21 -6.477) (size 1.778 1.778) (drill 1.016) (layers "*.Cu" "*.Mask") (remove_unused_layers no)
   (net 4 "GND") (solder_mask_margin 0.102))
  (pad "GND_2" thru_hole circle (at 29.083 -6.477) (size 1.778 1.778) (drill 1.016) (layers "*.Cu" "*.Mask") (remove_unused_layers no)
   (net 4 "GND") (solder_mask_margin 0.102))
  (pad "GND_3" thru_hole circle (at -24.13 11.303) (size 1.778 1.778) (drill 1) (layers "*.Cu" "*.Mask") (remove_unused_layers no)
   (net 4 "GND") (solder_mask_margin 0.102))
  (pad "GND_4" thru_hole circle (at -21.59 11.303) (size 1.778 1.778) (drill 1) (layers "*.Cu" "*.Mask") (remove_unused_layers no)
   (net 4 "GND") (solder_mask_margin 0.102))
  (pad "GND_5" thru_hole circle (at -19.05 11.303) (size 1.778 1.778) (drill 1) (layers "*.Cu" "*.Mask") (remove_unused_layers no)
   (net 4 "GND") (solder_mask_margin 0.102))
  (pad "GND_6" thru_hole circle (at -16.51 11.303) (size 1.778 1.778) (drill 1) (layers "*.Cu" "*.Mask") (remove_unused_layers no)
   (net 4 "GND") (solder_mask_margin 0.102))
  (pad "GND_7" thru_hole circle (at -11.43 11.303) (size 1.778 1.778) (drill 1) (layers "*.Cu" "*.Mask") (remove_unused_layers no)
   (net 4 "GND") (solder_mask_margin 0.102))
  (pad "GND_8" thru_hole circle (at -8.89 11.303) (size 1.778 1.778) (drill 1) (layers "*.Cu" "*.Mask") (remove_unused_layers no)
   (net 4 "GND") (solder_mask_margin 0.102))
  (pad "GND_9" thru_hole circle (at -6.35 11.303) (size 1.778 1.778) (drill 1) (layers "*.Cu" "*.Mask") (remove_unused_layers no)
   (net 4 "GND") (solder_mask_margin 0.102))
  (pad "GND_10" thru_hole circle (at -3.81 11.303) (size 1.778 1.778) (drill 1) (layers "*.Cu" "*.Mask") (remove_unused_layers no)
   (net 4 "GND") (solder_mask_margin 0.102))
  (pad "GND_11" thru_hole circle (at 3.81 11.303) (size 1.778 1.778) (drill 1) (layers "*.Cu" "*.Mask") (remove_unused_layers no)
   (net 4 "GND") (solder_mask_margin 0.102))
  (pad "GND_12" thru_hole circle (at 6.35 11.303) (size 1.778 1.778) (drill 1) (layers "*.Cu" "*.Mask") (remove_unused_layers no)
   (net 4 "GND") (solder_mask_margin 0.102))
  (pad "GND_13" thru_hole circle (at 8.89 11.303) (size 1.778 1.778) (drill 1) (layers "*.Cu" "*.Mask") (remove_unused_layers no)
   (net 4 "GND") (solder_mask_margin 0.102))
  (pad "GND_14" thru_hole circle (at 11.43 11.303) (size 1.778 1.778) (drill 1) (layers "*.Cu" "*.Mask") (remove_unused_layers no)
   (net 4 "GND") (solder_mask_margin 0.102))
  (pad "GND_15" thru_hole circle (at 16.51 11.303) (size 1.778 1.778) (drill 1) (layers "*.Cu" "*.Mask") (remove_unused_layers no)
   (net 4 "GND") (solder_mask_margin 0.102))
  (pad "GND_16" thru_hole circle (at 19.05 11.303) (size 1.778 1.778) (drill 1) (layers "*.Cu" "*.Mask") (remove_unused_layers no)
   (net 4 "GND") (solder_mask_margin 0.102))
  (pad "GND_17" thru_hole circle (at 21.59 11.303) (size 1.778 1.778) (drill 1) (layers "*.Cu" "*.Mask") (remove_unused_layers no)
   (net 4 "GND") (solder_mask_margin 0.102))
  (pad "GND_18" thru_hole circle (at 24.13 11.303) (size 1.778 1.778) (drill 1) (layers "*.Cu" "*.Mask") (remove_unused_layers no)
   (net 4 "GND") (solder_mask_margin 0.102))
  (pad "OE_1" thru_hole circle (at -29.21 -3.937) (size 1.778 1.778) (drill 1.016) (layers "*.Cu" "*.Mask") (remove_unused_layers no)
   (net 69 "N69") (solder_mask_margin 0.102))
  (pad "OE_2" thru_hole circle (at 29.083 -3.937) (size 1.778 1.778) (drill 1.016) (layers "*.Cu" "*.Mask") (remove_unused_layers no)
   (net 69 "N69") (solder_mask_margin 0.102))
  (pad "S1" thru_hole circle (at -27.94 -9.525) (size 3.2 3.2) (drill 2.5) (layers "*.Cu" "*.Mask") (remove_unused_layers no)
   (solder_mask_margin 0.102))
  (pad "S2" thru_hole circle (at 27.94 -9.525) (size 3.2 3.2) (drill 2.5) (layers "*.Cu" "*.Mask") (remove_unused_layers no)
   (solder_mask_margin 0.102))
  (pad "S3" thru_hole circle (at -27.94 9.525) (size 3.2 3.2) (drill 2.5) (layers "*.Cu" "*.Mask") (remove_unused_layers no)
   (solder_mask_margin 0.102))
  (pad "S4" thru_hole circle (at 27.94 9.525) (size 3.2 3.2) (drill 2.5) (layers "*.Cu" "*.Mask") (remove_unused_layers no)
   (solder_mask_margin 0.102))
  (pad "SCL_1" thru_hole circle (at -29.21 -1.397) (size 1.778 1.778) (drill 1.016) (layers "*.Cu" "*.Mask") (remove_unused_layers no)
   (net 24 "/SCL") (solder_mask_margin 0.102))
  (pad "SCL_2" thru_hole circle (at 29.083 -1.397) (size 1.778 1.778) (drill 1.016) (layers "*.Cu" "*.Mask") (remove_unused_layers no)
   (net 24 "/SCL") (solder_mask_margin 0.102))
  (pad "SDA_1" thru_hole circle (at -29.21 1.143) (size 1.778 1.778) (drill 1.016) (layers "*.Cu" "*.Mask") (remove_unused_layers no)
   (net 23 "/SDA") (solder_mask_margin 0.102))
  (pad "SDA_2" thru_hole circle (at 29.083 1.143) (size 1.778 1.778) (drill 1.016) (layers "*.Cu" "*.Mask") (remove_unused_layers no)
   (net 23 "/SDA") (solder_mask_margin 0.102))
  (pad "V+_1" thru_hole circle (at -29.21 6.223) (size 1.778 1.778) (drill 1.016) (layers "*.Cu" "*.Mask") (remove_unused_layers no)
   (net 49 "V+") (solder_mask_margin 0.102))
  (pad "V+_2" thru_hole circle (at 29.083 6.223) (size 1.778 1.778) (drill 1.016) (layers "*.Cu" "*.Mask") (remove_unused_layers no)
   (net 49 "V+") (solder_mask_margin 0.102))
  (pad "V+_3" thru_hole circle (at -24.13 8.763) (size 1.778 1.778) (drill 1) (layers "*.Cu" "*.Mask") (remove_unused_layers no)
   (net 49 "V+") (solder_mask_margin 0.102))
  (pad "V+_4" thru_hole circle (at -21.59 8.763) (size 1.778 1.778) (drill 1) (layers "*.Cu" "*.Mask") (remove_unused_layers no)
   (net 49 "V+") (solder_mask_margin 0.102))
  (pad "V+_5" thru_hole circle (at -19.05 8.763) (size 1.778 1.778) (drill 1) (layers "*.Cu" "*.Mask") (remove_unused_layers no)
   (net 49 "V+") (solder_mask_margin 0.102))
  (pad "V+_6" thru_hole circle (at -16.51 8.763) (size 1.778 1.778) (drill 1) (layers "*.Cu" "*.Mask") (remove_unused_layers no)
   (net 49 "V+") (solder_mask_margin 0.102))
  (pad "V+_7" thru_hole circle (at -11.43 8.763) (size 1.778 1.778) (drill 1) (layers "*.Cu" "*.Mask") (remove_unused_layers no)
   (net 49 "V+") (solder_mask_margin 0.102))
  (pad "V+_8" thru_hole circle (at -8.89 8.763) (size 1.778 1.778) (drill 1) (layers "*.Cu" "*.Mask") (remove_unused_layers no)
   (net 49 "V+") (solder_mask_margin 0.102))
  (pad "V+_9" thru_hole circle (at -6.35 8.763) (size 1.778 1.778) (drill 1) (layers "*.Cu" "*.Mask") (remove_unused_layers no)
   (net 49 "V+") (solder_mask_margin 0.102))
  (pad "V+_10" thru_hole circle (at -3.81 8.763) (size 1.778 1.778) (drill 1) (layers "*.Cu" "*.Mask") (remove_unused_layers no)
   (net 49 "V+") (solder_mask_margin 0.102))
  (pad "V+_11" thru_hole circle (at 3.81 8.763) (size 1.778 1.778) (drill 1) (layers "*.Cu" "*.Mask") (remove_unused_layers no)
   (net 49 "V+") (solder_mask_margin 0.102))
  (pad "V+_12" thru_hole circle (at 6.35 8.763) (size 1.778 1.778) (drill 1) (layers "*.Cu" "*.Mask") (remove_unused_layers no)
   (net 49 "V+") (solder_mask_margin 0.102))
  (pad "V+_13" thru_hole circle (at 8.89 8.763) (size 1.778 1.778) (drill 1) (layers "*.Cu" "*.Mask") (remove_unused_layers no)
   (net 49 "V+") (solder_mask_margin 0.102))
  (pad "V+_14" thru_hole circle (at 11.43 8.763) (size 1.778 1.778) (drill 1) (layers "*.Cu" "*.Mask") (remove_unused_layers no)
   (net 49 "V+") (solder_mask_margin 0.102))
  (pad "V+_15" thru_hole circle (at 16.51 8.763) (size 1.778 1.778) (drill 1) (layers "*.Cu" "*.Mask") (remove_unused_layers no)
   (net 49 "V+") (solder_mask_margin 0.102))
  (pad "V+_16" thru_hole circle (at 19.05 8.763) (size 1.778 1.778) (drill 1) (layers "*.Cu" "*.Mask") (remove_unused_layers no)
   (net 49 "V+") (solder_mask_margin 0.102))
  (pad "V+_17" thru_hole circle (at 21.59 8.763) (size 1.778 1.778) (drill 1) (layers "*.Cu" "*.Mask") (remove_unused_layers no)
   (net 49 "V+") (solder_mask_margin 0.102))
  (pad "V+_18" thru_hole circle (at 24.13 8.763) (size 1.778 1.778) (drill 1) (layers "*.Cu" "*.Mask") (remove_unused_layers no)
   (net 49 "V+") (solder_mask_margin 0.102))
  (pad "VCC_1" thru_hole circle (at -29.21 3.683) (size 1.778 1.778) (drill 1.016) (layers "*.Cu" "*.Mask") (remove_unused_layers no)
   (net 50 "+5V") (solder_mask_margin 0.102))
  (pad "VCC_2" thru_hole circle (at 29.083 3.683) (size 1.778 1.778) (drill 1.016) (layers "*.Cu" "*.Mask") (remove_unused_layers no)
   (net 50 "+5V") (solder_mask_margin 0.102)))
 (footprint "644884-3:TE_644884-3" (layer "F.Cu") (at 144.42 72.22)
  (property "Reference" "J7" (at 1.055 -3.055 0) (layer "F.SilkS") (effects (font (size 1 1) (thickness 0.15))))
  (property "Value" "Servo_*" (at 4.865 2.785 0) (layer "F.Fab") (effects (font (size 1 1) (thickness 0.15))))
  (pad "1" thru_hole rect (at 0 0) (size 1.37 1.37) (drill 1.02) (layers "*.Cu" "*.Mask") (remove_unused_layers no) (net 4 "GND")
   (solder_mask_margin 0.102))
  (pad "2" thru_hole circle (at 2.54 0) (size 1.37 1.37) (drill 1.02) (layers "*.Cu" "*.Mask") (remove_unused_layers no) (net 30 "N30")
   (solder_mask_margin 0.102))
  (pad "3" thru_hole circle (at 5.08 0) (size 1.37 1.37) (drill 1.02) (layers "*.Cu" "*.Mask") (remove_unused_layers no) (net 60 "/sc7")
   (solder_mask_margin 0.102)))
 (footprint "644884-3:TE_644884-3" (layer "F.Cu") (at 144.42 44.99)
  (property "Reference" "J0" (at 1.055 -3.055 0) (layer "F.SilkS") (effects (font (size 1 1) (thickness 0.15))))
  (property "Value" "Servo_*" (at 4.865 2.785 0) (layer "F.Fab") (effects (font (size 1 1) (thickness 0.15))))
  (pad "1" thru_hole rect (at 0 0) (size 1.37 1.37) (drill 1.02) (layers "*.Cu" "*.Mask") (remove_unused_layers no) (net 4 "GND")
   (solder_mask_margin 0.102))
  (pad "2" thru_hole circle (at 2.54 0) (size 1.37 1.37) (drill 1.02) (layers "*.Cu" "*.Mask") (remove_unused_layers no) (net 51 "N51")
   (solder_mask_margin 0.102))
  (pad "3" thru_hole circle (at 5.08 0) (size 1.37 1.37) (drill 1.02) (layers "*.Cu" "*.Mask") (remove_unused_layers no) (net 59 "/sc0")
   (solder_mask_margin 0.102)))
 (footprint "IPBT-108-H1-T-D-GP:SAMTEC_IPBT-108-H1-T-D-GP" (layer "F.Cu") (at 83.085 103.105)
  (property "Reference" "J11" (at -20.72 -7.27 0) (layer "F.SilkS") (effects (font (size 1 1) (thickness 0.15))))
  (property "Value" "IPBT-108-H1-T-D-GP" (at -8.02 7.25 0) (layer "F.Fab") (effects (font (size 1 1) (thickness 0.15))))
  (pad "01" thru_hole rect (at -14.665 -2.095) (size 2.13 2.13) (drill 1.78) (layers "*.Cu" "*.Mask") (remove_unused_layers no)
   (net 4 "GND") (solder_mask_margin 0.102))
  (pad "02" thru_hole circle (at -10.475 -2.095) (size 2.13 2.13) (drill 1.78) (layers "*.Cu" "*.Mask") (remove_unused_layers no)
   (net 50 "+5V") (solder_mask_margin 0.102))
  (pad "03" thru_hole circle (at -6.285 -2.095) (size 2.13 2.13) (drill 1.78) (layers "*.Cu" "*.Mask") (remove_unused_layers no)
   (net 32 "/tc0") (solder_mask_margin 0.102))
  (pad "04" thru_hole circle (at -2.095 -2.095) (size 2.13 2.13) (drill 1.78) (layers "*.Cu" "*.Mask") (remove_unused_layers no)
   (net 33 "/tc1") (solder_mask_margin 0.102))
  (pad "05" thru_hole circle (at 2.095 -2.095) (size 2.13 2.13) (drill 1.78) (layers "*.Cu" "*.Mask") (remove_unused_layers no)
   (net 34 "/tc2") (solder_mask_margin 0.102))
  (pad "06" thru_hole circle (at 6.285 -2.095) (size 2.13 2.13) (drill 1.78) (layers "*.Cu" "*.Mask") (remove_unused_layers no)
   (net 35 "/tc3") (solder_mask_margin 0.102))
  (pad "07" thru_hole circle (at 10.475 -2.095) (size 2.13 2.13) (drill 1.78) (layers "*.Cu" "*.Mask") (remove_unused_layers no)
   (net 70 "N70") (solder_mask_margin 0.102))
  (pad "08" thru_hole circle (at 14.665 -2.095) (size 2.13 2.13) (drill 1.78) (layers "*.Cu" "*.Mask") (remove_unused_layers no)
   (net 53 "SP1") (solder_mask_margin 0.102))
  (pad "09" thru_hole circle (at -14.665 2.095) (size 2.13 2.13) (drill 1.78) (layers "*.Cu" "*.Mask") (remove_unused_layers no)
   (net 4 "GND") (solder_mask_margin 0.102))
  (pad "10" thru_hole circle (at -10.475 2.095) (size 2.13 2.13) (drill 1.78) (layers "*.Cu" "*.Mask") (remove_unused_layers no)
   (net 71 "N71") (solder_mask_margin 0.102))
  (pad "11" thru_hole circle (at -6.285 2.095) (size 2.13 2.13) (drill 1.78) (layers "*.Cu" "*.Mask") (remove_unused_layers no)
   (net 36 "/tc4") (solder_mask_margin 0.102))
  (pad "12" thru_hole circle (at -2.095 2.095) (size 2.13 2.13) (drill 1.78) (layers "*.Cu" "*.Mask") (remove_unused_layers no)
   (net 37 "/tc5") (solder_mask_margin 0.102))
  (pad "13" thru_hole circle (at 2.095 2.095) (size 2.13 2.13) (drill 1.78) (layers "*.Cu" "*.Mask") (remove_unused_layers no)
   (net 38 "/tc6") (solder_mask_margin 0.102))
  (pad "14" thru_hole circle (at 6.285 2.095) (size 2.13 2.13) (drill 1.78) (layers "*.Cu" "*.Mask") (remove_unused_layers no)
   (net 39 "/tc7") (solder_mask_margin 0.102))
  (pad "15" thru_hole circle (at 10.475 2.095) (size 2.13 2.13) (drill 1.78) (layers "*.Cu" "*.Mask") (remove_unused_layers no)
   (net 4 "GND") (solder_mask_margin 0.102))
  (pad "16" thru_hole circle (at 14.665 2.095) (size 2.13 2.13) (drill 1.78) (layers "*.Cu" "*.Mask") (remove_unused_layers no)
   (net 54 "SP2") (solder_mask_margin 0.102)))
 (gr_rect (start 48.5 38.5) (end 168.5 120) (stroke (width 0.05) (type default)) (fill no) (layer "Edge.Cuts"))
 (segment (start 61.52 89.693) (end 62.17642 89.693) (width 0.2) (layer "F.Cu") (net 49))
 (segment (start 117.4 89.693) (end 114.86 92.233) (width 0.2) (layer "F.Cu") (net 49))
 (segment (start 64.71642 92.233) (end 114.86 92.233) (width 0.2) (layer "F.Cu") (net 49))
 (segment (start 62.17642 89.693) (end 64.71642 92.233) (width 0.2) (layer "F.Cu") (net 49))
 (segment (start 119.813 89.693) (end 117.4 89.693) (width 0.2) (layer "F.Cu") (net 49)))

